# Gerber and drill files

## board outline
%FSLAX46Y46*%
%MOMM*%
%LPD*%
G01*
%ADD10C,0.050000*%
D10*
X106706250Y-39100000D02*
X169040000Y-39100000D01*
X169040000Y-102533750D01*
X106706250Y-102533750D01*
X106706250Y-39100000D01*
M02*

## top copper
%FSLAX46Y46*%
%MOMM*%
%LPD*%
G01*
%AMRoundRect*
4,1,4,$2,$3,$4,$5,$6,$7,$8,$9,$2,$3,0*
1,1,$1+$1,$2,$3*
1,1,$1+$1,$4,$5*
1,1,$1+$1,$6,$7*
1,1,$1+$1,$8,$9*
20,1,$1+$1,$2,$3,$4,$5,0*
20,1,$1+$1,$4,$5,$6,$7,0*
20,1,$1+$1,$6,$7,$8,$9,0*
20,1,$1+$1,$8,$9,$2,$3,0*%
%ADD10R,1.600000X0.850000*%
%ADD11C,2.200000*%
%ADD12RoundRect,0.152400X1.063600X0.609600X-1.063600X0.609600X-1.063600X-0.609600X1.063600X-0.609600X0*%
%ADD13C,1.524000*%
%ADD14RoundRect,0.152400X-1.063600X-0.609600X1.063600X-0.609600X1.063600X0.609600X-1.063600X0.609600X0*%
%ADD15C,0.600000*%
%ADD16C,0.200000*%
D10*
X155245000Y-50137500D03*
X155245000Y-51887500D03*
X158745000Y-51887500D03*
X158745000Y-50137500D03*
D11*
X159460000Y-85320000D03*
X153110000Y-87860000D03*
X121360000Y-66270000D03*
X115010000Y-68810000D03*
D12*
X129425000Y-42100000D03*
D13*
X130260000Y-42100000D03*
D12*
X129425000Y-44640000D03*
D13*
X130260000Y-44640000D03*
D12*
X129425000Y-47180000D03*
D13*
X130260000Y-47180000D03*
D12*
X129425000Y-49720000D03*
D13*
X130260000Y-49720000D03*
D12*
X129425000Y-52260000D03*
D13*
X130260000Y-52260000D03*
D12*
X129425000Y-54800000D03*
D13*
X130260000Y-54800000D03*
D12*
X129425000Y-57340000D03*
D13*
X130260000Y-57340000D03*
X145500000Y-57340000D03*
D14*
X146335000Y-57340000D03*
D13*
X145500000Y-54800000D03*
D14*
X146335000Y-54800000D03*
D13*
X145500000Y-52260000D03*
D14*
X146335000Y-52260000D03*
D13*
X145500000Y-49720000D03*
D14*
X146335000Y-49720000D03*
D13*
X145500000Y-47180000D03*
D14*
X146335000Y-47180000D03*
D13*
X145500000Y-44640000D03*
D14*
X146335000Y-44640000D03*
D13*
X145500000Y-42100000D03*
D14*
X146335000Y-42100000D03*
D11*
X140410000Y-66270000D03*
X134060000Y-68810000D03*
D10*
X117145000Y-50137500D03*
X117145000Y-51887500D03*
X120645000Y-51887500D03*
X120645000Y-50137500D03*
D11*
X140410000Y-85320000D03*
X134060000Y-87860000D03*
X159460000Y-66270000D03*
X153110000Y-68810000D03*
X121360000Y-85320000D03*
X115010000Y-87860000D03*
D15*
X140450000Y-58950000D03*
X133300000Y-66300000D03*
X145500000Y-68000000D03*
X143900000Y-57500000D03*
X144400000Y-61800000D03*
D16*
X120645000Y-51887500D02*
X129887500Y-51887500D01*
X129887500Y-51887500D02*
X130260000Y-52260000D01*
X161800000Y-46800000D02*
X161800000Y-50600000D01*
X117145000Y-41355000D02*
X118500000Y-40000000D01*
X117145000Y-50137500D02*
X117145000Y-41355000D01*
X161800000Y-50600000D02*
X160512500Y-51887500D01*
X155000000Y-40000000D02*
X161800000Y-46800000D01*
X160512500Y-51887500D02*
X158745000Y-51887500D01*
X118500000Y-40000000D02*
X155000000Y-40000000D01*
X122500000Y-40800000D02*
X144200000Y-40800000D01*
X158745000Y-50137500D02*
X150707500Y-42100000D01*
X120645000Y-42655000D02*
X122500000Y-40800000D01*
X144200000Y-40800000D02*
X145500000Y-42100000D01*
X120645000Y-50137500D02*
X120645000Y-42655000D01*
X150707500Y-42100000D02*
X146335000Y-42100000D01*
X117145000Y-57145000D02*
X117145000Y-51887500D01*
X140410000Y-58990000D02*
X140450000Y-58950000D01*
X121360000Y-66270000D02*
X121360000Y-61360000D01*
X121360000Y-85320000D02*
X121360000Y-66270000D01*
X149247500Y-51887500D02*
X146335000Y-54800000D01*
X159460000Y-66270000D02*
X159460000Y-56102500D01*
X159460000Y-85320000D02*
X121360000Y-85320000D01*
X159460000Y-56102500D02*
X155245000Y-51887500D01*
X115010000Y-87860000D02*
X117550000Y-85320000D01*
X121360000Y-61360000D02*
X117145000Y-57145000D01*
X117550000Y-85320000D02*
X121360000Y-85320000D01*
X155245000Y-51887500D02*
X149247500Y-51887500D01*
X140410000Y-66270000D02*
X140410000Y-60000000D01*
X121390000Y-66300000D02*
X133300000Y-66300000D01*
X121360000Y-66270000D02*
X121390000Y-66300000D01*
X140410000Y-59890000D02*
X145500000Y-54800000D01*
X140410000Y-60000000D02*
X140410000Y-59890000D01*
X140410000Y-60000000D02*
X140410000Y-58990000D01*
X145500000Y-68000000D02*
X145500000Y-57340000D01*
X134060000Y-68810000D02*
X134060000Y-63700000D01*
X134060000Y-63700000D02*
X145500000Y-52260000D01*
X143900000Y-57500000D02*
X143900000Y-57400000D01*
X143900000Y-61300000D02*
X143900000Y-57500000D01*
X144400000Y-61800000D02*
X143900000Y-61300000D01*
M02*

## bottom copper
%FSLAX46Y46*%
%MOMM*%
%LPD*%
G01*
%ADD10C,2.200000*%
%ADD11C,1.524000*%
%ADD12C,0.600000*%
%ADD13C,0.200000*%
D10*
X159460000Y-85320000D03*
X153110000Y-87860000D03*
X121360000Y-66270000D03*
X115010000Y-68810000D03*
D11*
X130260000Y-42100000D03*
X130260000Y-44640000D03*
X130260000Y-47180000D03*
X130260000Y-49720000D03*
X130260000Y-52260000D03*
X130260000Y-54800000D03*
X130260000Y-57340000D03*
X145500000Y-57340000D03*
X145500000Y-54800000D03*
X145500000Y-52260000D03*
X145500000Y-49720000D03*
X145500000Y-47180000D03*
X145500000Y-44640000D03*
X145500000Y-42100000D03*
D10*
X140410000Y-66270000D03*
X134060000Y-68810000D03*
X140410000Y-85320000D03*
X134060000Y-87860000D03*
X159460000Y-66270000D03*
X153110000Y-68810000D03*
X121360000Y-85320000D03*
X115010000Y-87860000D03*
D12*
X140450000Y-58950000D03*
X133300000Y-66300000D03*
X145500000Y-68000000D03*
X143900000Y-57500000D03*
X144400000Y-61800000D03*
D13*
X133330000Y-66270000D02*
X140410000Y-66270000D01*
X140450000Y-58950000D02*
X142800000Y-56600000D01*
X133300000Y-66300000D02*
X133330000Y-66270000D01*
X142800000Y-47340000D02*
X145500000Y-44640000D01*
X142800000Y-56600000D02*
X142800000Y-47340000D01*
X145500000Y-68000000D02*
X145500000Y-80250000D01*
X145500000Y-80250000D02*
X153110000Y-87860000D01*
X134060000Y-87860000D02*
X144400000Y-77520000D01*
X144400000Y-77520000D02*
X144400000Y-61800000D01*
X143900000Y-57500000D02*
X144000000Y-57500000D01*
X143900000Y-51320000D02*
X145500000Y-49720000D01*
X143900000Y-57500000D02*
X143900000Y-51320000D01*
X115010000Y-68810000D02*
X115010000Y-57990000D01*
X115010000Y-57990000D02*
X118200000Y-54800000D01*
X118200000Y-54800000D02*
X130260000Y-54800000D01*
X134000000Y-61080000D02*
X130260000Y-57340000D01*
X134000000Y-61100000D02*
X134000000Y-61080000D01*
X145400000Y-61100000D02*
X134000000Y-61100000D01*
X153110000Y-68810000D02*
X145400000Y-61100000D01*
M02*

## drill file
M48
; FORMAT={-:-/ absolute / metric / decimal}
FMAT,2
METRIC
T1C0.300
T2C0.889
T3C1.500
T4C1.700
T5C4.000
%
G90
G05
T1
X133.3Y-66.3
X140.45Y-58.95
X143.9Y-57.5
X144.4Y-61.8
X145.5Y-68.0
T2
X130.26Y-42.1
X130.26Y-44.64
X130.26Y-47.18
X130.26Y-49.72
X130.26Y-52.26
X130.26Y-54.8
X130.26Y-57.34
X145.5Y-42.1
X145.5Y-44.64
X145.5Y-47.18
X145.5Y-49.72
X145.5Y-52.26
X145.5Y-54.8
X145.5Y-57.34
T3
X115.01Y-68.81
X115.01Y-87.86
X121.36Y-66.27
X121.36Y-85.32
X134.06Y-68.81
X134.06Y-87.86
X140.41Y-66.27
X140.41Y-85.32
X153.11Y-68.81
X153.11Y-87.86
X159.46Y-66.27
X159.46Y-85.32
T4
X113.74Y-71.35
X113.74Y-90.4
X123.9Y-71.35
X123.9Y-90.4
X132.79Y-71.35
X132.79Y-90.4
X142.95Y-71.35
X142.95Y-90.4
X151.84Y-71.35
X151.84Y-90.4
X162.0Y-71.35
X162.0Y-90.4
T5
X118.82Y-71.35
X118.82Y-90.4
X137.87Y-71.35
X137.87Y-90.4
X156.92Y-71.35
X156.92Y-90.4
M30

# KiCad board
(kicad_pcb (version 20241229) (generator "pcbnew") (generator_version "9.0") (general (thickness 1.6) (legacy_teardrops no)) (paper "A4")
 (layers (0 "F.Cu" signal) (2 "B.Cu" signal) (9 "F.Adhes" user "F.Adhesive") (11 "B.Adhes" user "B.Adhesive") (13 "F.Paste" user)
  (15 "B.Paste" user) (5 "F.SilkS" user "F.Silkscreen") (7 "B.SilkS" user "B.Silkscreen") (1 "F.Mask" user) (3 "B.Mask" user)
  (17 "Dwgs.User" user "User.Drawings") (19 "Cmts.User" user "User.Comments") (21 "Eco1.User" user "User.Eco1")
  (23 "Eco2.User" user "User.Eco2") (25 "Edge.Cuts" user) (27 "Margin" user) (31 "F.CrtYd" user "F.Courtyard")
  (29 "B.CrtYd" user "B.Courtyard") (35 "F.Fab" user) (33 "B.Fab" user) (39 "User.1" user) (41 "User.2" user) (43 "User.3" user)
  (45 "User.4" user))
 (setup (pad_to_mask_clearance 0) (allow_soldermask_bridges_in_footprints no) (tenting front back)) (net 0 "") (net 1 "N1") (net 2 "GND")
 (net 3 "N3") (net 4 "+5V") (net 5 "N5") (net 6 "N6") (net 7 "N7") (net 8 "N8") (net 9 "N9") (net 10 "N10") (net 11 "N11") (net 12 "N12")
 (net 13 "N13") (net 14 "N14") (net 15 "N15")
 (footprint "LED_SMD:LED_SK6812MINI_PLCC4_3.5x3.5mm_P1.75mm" (layer "F.Cu") (at 156.995 51.0125)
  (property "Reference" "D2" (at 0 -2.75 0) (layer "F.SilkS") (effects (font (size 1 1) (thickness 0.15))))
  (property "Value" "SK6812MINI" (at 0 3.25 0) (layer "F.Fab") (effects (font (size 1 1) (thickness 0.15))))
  (pad "1" smd rect (at -1.75 -0.875) (size 1.6 0.85) (layers "F.Cu" "F.Mask" "F.Paste") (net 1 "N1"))
  (pad "2" smd rect (at -1.75 0.875) (size 1.6 0.85) (layers "F.Cu" "F.Mask" "F.Paste") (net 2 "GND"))
  (pad "3" smd rect (at 1.75 0.875) (size 1.6 0.85) (layers "F.Cu" "F.Mask" "F.Paste") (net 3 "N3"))
  (pad "4" smd rect (at 1.75 -0.875) (size 1.6 0.85) (layers "F.Cu" "F.Mask" "F.Paste") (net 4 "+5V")))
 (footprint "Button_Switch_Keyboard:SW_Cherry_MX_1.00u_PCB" (layer "F.Cu") (at 159.46 85.32)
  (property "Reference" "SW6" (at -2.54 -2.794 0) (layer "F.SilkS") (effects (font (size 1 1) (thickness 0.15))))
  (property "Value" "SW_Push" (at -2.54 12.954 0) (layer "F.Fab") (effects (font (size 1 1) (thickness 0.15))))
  (pad "" np_thru_hole circle (at -7.62 5.08) (size 1.7 1.7) (drill 1.7) (layers "*.Cu" "*.Mask"))
  (pad "" np_thru_hole circle (at -2.54 5.08) (size 4 4) (drill 4) (layers "*.Cu" "*.Mask"))
  (pad "" np_thru_hole circle (at 2.54 5.08) (size 1.7 1.7) (drill 1.7) (layers "*.Cu" "*.Mask"))
  (pad "1" thru_hole circle (at 0 0) (size 2.2 2.2) (drill 1.5) (layers "*.Cu" "*.Mask") (remove_unused_layers no) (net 2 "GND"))
  (pad "2" thru_hole circle (at -6.35 2.54) (size 2.2 2.2) (drill 1.5) (layers "*.Cu" "*.Mask") (remove_unused_layers no) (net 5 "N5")))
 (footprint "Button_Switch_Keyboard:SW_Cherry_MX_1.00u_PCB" (layer "F.Cu") (at 121.36 66.27)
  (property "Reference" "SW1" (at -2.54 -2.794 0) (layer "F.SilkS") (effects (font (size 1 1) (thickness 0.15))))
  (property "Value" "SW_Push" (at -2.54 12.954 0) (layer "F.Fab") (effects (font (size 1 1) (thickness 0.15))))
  (pad "" np_thru_hole circle (at -7.62 5.08) (size 1.7 1.7) (drill 1.7) (layers "*.Cu" "*.Mask"))
  (pad "" np_thru_hole circle (at -2.54 5.08) (size 4 4) (drill 4) (layers "*.Cu" "*.Mask"))
  (pad "" np_thru_hole circle (at 2.54 5.08) (size 1.7 1.7) (drill 1.7) (layers "*.Cu" "*.Mask"))
  (pad "1" thru_hole circle (at 0 0) (size 2.2 2.2) (drill 1.5) (layers "*.Cu" "*.Mask") (remove_unused_layers no) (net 2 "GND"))
  (pad "2" thru_hole circle (at -6.35 2.54) (size 2.2 2.2) (drill 1.5) (layers "*.Cu" "*.Mask") (remove_unused_layers no) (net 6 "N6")))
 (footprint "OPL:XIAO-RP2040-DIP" (layer "F.Cu") (at 137.88 49.72)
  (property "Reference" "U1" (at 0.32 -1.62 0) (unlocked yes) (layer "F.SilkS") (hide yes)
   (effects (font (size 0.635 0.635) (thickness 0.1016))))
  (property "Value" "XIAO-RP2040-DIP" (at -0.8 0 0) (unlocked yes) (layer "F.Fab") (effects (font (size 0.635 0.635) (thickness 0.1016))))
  (pad "1" smd roundrect (at -8.455 -7.62 180) (size 2.432 1.524) (layers "F.Cu" "F.Mask") (roundrect_rratio 0.1) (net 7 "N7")
   (thermal_bridge_angle 45))
  (pad "1" thru_hole circle (at -7.62 -7.62 180) (size 1.524 1.524) (drill 0.889) (layers "*.Cu" "*.Mask") (remove_unused_layers no)
   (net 7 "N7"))
  (pad "2" smd roundrect (at -8.455 -5.08 180) (size 2.432 1.524) (layers "F.Cu" "F.Mask") (roundrect_rratio 0.1) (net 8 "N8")
   (thermal_bridge_angle 45))
  (pad "2" thru_hole circle (at -7.62 -5.08 180) (size 1.524 1.524) (drill 0.889) (layers "*.Cu" "*.Mask") (remove_unused_layers no)
   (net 8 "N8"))
  (pad "3" smd roundrect (at -8.455 -2.54 180) (size 2.432 1.524) (layers "F.Cu" "F.Mask") (roundrect_rratio 0.1) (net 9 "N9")
   (thermal_bridge_angle 45))
  (pad "3" thru_hole circle (at -7.62 -2.54 180) (size 1.524 1.524) (drill 0.889) (layers "*.Cu" "*.Mask") (remove_unused_layers no)
   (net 9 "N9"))
  (pad "4" smd roundrect (at -8.455 0 180) (size 2.432 1.524) (layers "F.Cu" "F.Mask") (roundrect_rratio 0.1) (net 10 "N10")
   (thermal_bridge_angle 45))
  (pad "4" thru_hole circle (at -7.62 0 180) (size 1.524 1.524) (drill 0.889) (layers "*.Cu" "*.Mask") (remove_unused_layers no)
   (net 10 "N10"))
  (pad "5" smd roundrect (at -8.455 2.54 180) (size 2.432 1.524) (layers "F.Cu" "F.Mask") (roundrect_rratio 0.1) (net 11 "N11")
   (thermal_bridge_angle 45))
  (pad "5" thru_hole circle (at -7.62 2.54 180) (size 1.524 1.524) (drill 0.889) (layers "*.Cu" "*.Mask") (remove_unused_layers no)
   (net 11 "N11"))
  (pad "6" smd roundrect (at -8.455 5.08 180) (size 2.432 1.524) (layers "F.Cu" "F.Mask") (roundrect_rratio 0.1) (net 6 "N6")
   (thermal_bridge_angle 45))
  (pad "6" thru_hole circle (at -7.62 5.08 180) (size 1.524 1.524) (drill 0.889) (layers "*.Cu" "*.Mask") (remove_unused_layers no)
   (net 6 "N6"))
  (pad "7" smd roundrect (at -8.455 7.62 180) (size 2.432 1.524) (layers "F.Cu" "F.Mask") (roundrect_rratio 0.1) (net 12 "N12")
   (thermal_bridge_angle 45))
  (pad "7" thru_hole circle (at -7.62 7.62 180) (size 1.524 1.524) (drill 0.889) (layers "*.Cu" "*.Mask") (remove_unused_layers no)
   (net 12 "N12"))
  (pad "8" thru_hole circle (at 7.62 7.62) (size 1.524 1.524) (drill 0.889) (layers "*.Cu" "*.Mask") (remove_unused_layers no) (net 5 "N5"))
  (pad "8" smd roundrect (at 8.455 7.62) (size 2.432 1.524) (layers "F.Cu" "F.Mask") (roundrect_rratio 0.1) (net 5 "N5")
   (thermal_bridge_angle 45))
  (pad "9" thru_hole circle (at 7.62 5.08) (size 1.524 1.524) (drill 0.889) (layers "*.Cu" "*.Mask") (remove_unused_layers no) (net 2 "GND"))
  (pad "9" smd roundrect (at 8.455 5.08) (size 2.432 1.524) (layers "F.Cu" "F.Mask") (roundrect_rratio 0.1) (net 2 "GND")
   (thermal_bridge_angle 45))
  (pad "10" thru_hole circle (at 7.62 2.54) (size 1.524 1.524) (drill 0.889) (layers "*.Cu" "*.Mask") (remove_unused_layers no)
   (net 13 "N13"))
  (pad "10" smd roundrect (at 8.455 2.54) (size 2.432 1.524) (layers "F.Cu" "F.Mask") (roundrect_rratio 0.1) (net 13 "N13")
   (thermal_bridge_angle 45))
  (pad "11" thru_hole circle (at 7.62 0) (size 1.524 1.524) (drill 0.889) (layers "*.Cu" "*.Mask") (remove_unused_layers no) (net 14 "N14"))
  (pad "11" smd roundrect (at 8.455 0) (size 2.432 1.524) (layers "F.Cu" "F.Mask") (roundrect_rratio 0.1) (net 14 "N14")
   (thermal_bridge_angle 45))
  (pad "12" thru_hole circle (at 7.62 -2.54) (size 1.524 1.524) (drill 0.889) (layers "*.Cu" "*.Mask") (remove_unused_layers no)
   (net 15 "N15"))
  (pad "12" smd roundrect (at 8.455 -2.54) (size 2.432 1.524) (layers "F.Cu" "F.Mask") (roundrect_rratio 0.1) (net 15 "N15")
   (thermal_bridge_angle 45))
  (pad "13" thru_hole circle (at 7.62 -5.08) (size 1.524 1.524) (drill 0.889) (layers "*.Cu" "*.Mask") (remove_unused_layers no)
   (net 2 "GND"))
  (pad "13" smd roundrect (at 8.455 -5.08) (size 2.432 1.524) (layers "F.Cu" "F.Mask") (roundrect_rratio 0.1) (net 2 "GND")
   (thermal_bridge_angle 45))
  (pad "14" thru_hole circle (at 7.62 -7.62) (size 1.524 1.524) (drill 0.889) (layers "*.Cu" "*.Mask") (remove_unused_layers no)
   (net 4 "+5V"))
  (pad "14" smd roundrect (at 8.455 -7.62) (size 2.432 1.524) (layers "F.Cu" "F.Mask") (roundrect_rratio 0.1) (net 4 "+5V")
   (thermal_bridge_angle 45)))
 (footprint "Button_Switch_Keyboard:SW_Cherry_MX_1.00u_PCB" (layer "F.Cu") (at 140.41 66.27)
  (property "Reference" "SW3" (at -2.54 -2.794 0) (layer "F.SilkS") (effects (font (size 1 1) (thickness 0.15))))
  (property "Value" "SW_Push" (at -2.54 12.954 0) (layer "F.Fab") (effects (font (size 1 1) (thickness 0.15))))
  (pad "" np_thru_hole circle (at -7.62 5.08) (size 1.7 1.7) (drill 1.7) (layers "*.Cu" "*.Mask"))
  (pad "" np_thru_hole circle (at -2.54 5.08) (size 4 4) (drill 4) (layers "*.Cu" "*.Mask"))
  (pad "" np_thru_hole circle (at 2.54 5.08) (size 1.7 1.7) (drill 1.7) (layers "*.Cu" "*.Mask"))
  (pad "1" thru_hole circle (at 0 0) (size 2.2 2.2) (drill 1.5) (layers "*.Cu" "*.Mask") (remove_unused_layers no) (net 2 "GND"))
  (pad "2" thru_hole circle (at -6.35 2.54) (size 2.2 2.2) (drill 1.5) (layers "*.Cu" "*.Mask") (remove_unused_layers no) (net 13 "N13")))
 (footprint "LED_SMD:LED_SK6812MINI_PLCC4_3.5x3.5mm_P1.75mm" (layer "F.Cu") (at 118.895 51.0125)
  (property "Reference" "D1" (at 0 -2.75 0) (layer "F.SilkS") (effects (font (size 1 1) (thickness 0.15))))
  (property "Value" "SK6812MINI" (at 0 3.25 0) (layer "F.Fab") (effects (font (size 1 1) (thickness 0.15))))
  (pad "1" smd rect (at -1.75 -0.875) (size 1.6 0.85) (layers "F.Cu" "F.Mask" "F.Paste") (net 3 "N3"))
  (pad "2" smd rect (at -1.75 0.875) (size 1.6 0.85) (layers "F.Cu" "F.Mask" "F.Paste") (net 2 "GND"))
  (pad "3" smd rect (at 1.75 0.875) (size 1.6 0.85) (layers "F.Cu" "F.Mask" "F.Paste") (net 11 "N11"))
  (pad "4" smd rect (at 1.75 -0.875) (size 1.6 0.85) (layers "F.Cu" "F.Mask" "F.Paste") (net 4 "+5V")))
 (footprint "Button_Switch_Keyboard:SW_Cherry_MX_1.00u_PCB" (layer "F.Cu") (at 140.41 85.32)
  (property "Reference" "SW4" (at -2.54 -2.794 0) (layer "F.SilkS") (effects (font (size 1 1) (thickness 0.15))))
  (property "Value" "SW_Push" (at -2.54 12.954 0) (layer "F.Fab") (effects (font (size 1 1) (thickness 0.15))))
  (pad "" np_thru_hole circle (at -7.62 5.08) (size 1.7 1.7) (drill 1.7) (layers "*.Cu" "*.Mask"))
  (pad "" np_thru_hole circle (at -2.54 5.08) (size 4 4) (drill 4) (layers "*.Cu" "*.Mask"))
  (pad "" np_thru_hole circle (at 2.54 5.08) (size 1.7 1.7) (drill 1.7) (layers "*.Cu" "*.Mask"))
  (pad "1" thru_hole circle (at 0 0) (size 2.2 2.2) (drill 1.5) (layers "*.Cu" "*.Mask") (remove_unused_layers no) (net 2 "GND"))
  (pad "2" thru_hole circle (at -6.35 2.54) (size 2.2 2.2) (drill 1.5) (layers "*.Cu" "*.Mask") (remove_unused_layers no) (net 14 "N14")))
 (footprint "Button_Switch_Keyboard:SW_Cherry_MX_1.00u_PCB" (layer "F.Cu") (at 159.46 66.27)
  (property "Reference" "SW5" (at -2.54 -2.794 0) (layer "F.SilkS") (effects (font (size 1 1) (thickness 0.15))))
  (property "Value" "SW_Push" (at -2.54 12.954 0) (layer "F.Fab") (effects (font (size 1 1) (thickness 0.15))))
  (pad "" np_thru_hole circle (at -7.62 5.08) (size 1.7 1.7) (drill 1.7) (layers "*.Cu" "*.Mask"))
  (pad "" np_thru_hole circle (at -2.54 5.08) (size 4 4) (drill 4) (layers "*.Cu" "*.Mask"))
  (pad "" np_thru_hole circle (at 2.54 5.08) (size 1.7 1.7) (drill 1.7) (layers "*.Cu" "*.Mask"))
  (pad "1" thru_hole circle (at 0 0) (size 2.2 2.2) (drill 1.5) (layers "*.Cu" "*.Mask") (remove_unused_layers no) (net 2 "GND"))
  (pad "2" thru_hole circle (at -6.35 2.54) (size 2.2 2.2) (drill 1.5) (layers "*.Cu" "*.Mask") (remove_unused_layers no) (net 12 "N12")))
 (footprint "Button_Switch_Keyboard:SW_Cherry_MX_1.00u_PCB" (layer "F.Cu") (at 121.36 85.32)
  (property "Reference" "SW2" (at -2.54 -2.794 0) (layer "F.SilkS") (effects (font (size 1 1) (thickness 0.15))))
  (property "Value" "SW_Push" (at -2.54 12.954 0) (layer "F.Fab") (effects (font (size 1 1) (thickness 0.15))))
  (pad "" np_thru_hole circle (at -7.62 5.08) (size 1.7 1.7) (drill 1.7) (layers "*.Cu" "*.Mask"))
  (pad "" np_thru_hole circle (at -2.54 5.08) (size 4 4) (drill 4) (layers "*.Cu" "*.Mask"))
  (pad "" np_thru_hole circle (at 2.54 5.08) (size 1.7 1.7) (drill 1.7) (layers "*.Cu" "*.Mask"))
  (pad "1" thru_hole circle (at 0 0) (size 2.2 2.2) (drill 1.5) (layers "*.Cu" "*.Mask") (remove_unused_layers no) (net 2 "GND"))
  (pad "2" thru_hole circle (at -6.35 2.54) (size 2.2 2.2) (drill 1.5) (layers "*.Cu" "*.Mask") (remove_unused_layers no) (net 2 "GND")))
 (gr_rect (start 106.70625 39.1) (end 169.04 102.53375) (stroke (width 0.05) (type default)) (fill no) (layer "Edge.Cuts"))
 (segment (start 120.645 51.8875) (end 129.8875 51.8875) (width 0.2) (layer "F.Cu") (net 11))
 (segment (start 129.8875 51.8875) (end 130.26 52.26) (width 0.2) (layer "F.Cu") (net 11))
 (segment (start 161.8 46.8) (end 161.8 50.6) (width 0.2) (layer "F.Cu") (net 3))
 (segment (start 117.145 41.355) (end 118.5 40) (width 0.2) (layer "F.Cu") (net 3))
 (segment (start 117.145 50.1375) (end 117.145 41.355) (width 0.2) (layer "F.Cu") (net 3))
 (segment (start 161.8 50.6) (end 160.5125 51.8875) (width 0.2) (layer "F.Cu") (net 3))
 (segment (start 155 40) (end 161.8 46.8) (width 0.2) (layer "F.Cu") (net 3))
 (segment (start 160.5125 51.8875) (end 158.745 51.8875) (width 0.2) (layer "F.Cu") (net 3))
 (segment (start 118.5 40) (end 155 40) (width 0.2) (layer "F.Cu") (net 3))
 (segment (start 122.5 40.8) (end 144.2 40.8) (width 0.2) (layer "F.Cu") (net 4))
 (segment (start 158.745 50.1375) (end 150.7075 42.1) (width 0.2) (layer "F.Cu") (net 4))
 (segment (start 120.645 42.655) (end 122.5 40.8) (width 0.2) (layer "F.Cu") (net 4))
 (segment (start 144.2 40.8) (end 145.5 42.1) (width 0.2) (layer "F.Cu") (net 4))
 (segment (start 120.645 50.1375) (end 120.645 42.655) (width 0.2) (layer "F.Cu") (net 4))
 (segment (start 150.7075 42.1) (end 146.335 42.1) (width 0.2) (layer "F.Cu") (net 4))
 (segment (start 117.145 57.145) (end 117.145 51.8875) (width 0.2) (layer "F.Cu") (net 2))
 (segment (start 140.41 58.99) (end 140.45 58.95) (width 0.2) (layer "F.Cu") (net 2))
 (segment (start 121.36 66.27) (end 121.36 61.36) (width 0.2) (layer "F.Cu") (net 2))
 (segment (start 121.36 85.32) (end 121.36 66.27) (width 0.2) (layer "F.Cu") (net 2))
 (segment (start 149.2475 51.8875) (end 146.335 54.8) (width 0.2) (layer "F.Cu") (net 2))
 (segment (start 159.46 66.27) (end 159.46 56.1025) (width 0.2) (layer "F.Cu") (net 2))
 (segment (start 159.46 85.32) (end 121.36 85.32) (width 0.2) (layer "F.Cu") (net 2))
 (segment (start 159.46 56.1025) (end 155.245 51.8875) (width 0.2) (layer "F.Cu") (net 2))
 (segment (start 115.01 87.86) (end 117.55 85.32) (width 0.2) (layer "F.Cu") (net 2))
 (segment (start 121.36 61.36) (end 117.145 57.145) (width 0.2) (layer "F.Cu") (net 2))
 (segment (start 117.55 85.32) (end 121.36 85.32) (width 0.2) (layer "F.Cu") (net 2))
 (segment (start 155.245 51.8875) (end 149.2475 51.8875) (width 0.2) (layer "F.Cu") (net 2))
 (segment (start 140.41 66.27) (end 140.41 60) (width 0.2) (layer "F.Cu") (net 2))
 (segment (start 121.39 66.3) (end 133.3 66.3) (width 0.2) (layer "F.Cu") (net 2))
 (segment (start 121.36 66.27) (end 121.39 66.3) (width 0.2) (layer "F.Cu") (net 2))
 (segment (start 140.41 59.89) (end 145.5 54.8) (width 0.2) (layer "F.Cu") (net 2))
 (segment (start 140.41 60) (end 140.41 59.89) (width 0.2) (layer "F.Cu") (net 2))
 (segment (start 140.41 60) (end 140.41 58.99) (width 0.2) (layer "F.Cu") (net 2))
 (via (at 140.45 58.95) (size 0.6) (drill 0.3) (layers "F.Cu" "B.Cu") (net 2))
 (via (at 133.3 66.3) (size 0.6) (drill 0.3) (layers "F.Cu" "B.Cu") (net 2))
 (segment (start 133.33 66.27) (end 140.41 66.27) (width 0.2) (layer "B.Cu") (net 2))
 (segment (start 140.45 58.95) (end 142.8 56.6) (width 0.2) (layer "B.Cu") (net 2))
 (segment (start 133.3 66.3) (end 133.33 66.27) (width 0.2) (layer "B.Cu") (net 2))
 (segment (start 142.8 47.34) (end 145.5 44.64) (width 0.2) (layer "B.Cu") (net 2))
 (segment (start 142.8 56.6) (end 142.8 47.34) (width 0.2) (layer "B.Cu") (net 2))
 (segment (start 145.5 68) (end 145.5 57.34) (width 0.2) (layer "F.Cu") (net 5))
 (via (at 145.5 68) (size 0.6) (drill 0.3) (layers "F.Cu" "B.Cu") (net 5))
 (segment (start 145.5 68) (end 145.5 80.25) (width 0.2) (layer "B.Cu") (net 5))
 (segment (start 145.5 80.25) (end 153.11 87.86) (width 0.2) (layer "B.Cu") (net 5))
 (segment (start 134.06 68.81) (end 134.06 63.7) (width 0.2) (layer "F.Cu") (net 13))
 (segment (start 134.06 63.7) (end 145.5 52.26) (width 0.2) (layer "F.Cu") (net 13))
 (segment (start 143.9 57.5) (end 143.9 57.4) (width 0.2) (layer "F.Cu") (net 14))
 (segment (start 143.9 61.3) (end 143.9 57.5) (width 0.2) (layer "F.Cu") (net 14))
 (segment (start 144.4 61.8) (end 143.9 61.3) (width 0.2) (layer "F.Cu") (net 14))
 (via (at 143.9 57.5) (size 0.6) (drill 0.3) (layers "F.Cu" "B.Cu") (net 14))
 (via (at 144.4 61.8) (size 0.6) (drill 0.3) (layers "F.Cu" "B.Cu") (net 14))
 (segment (start 134.06 87.86) (end 144.4 77.52) (width 0.2) (layer "B.Cu") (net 14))
 (segment (start 144.4 77.52) (end 144.4 61.8) (width 0.2) (layer "B.Cu") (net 14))
 (segment (start 143.9 57.5) (end 144 57.5) (width 0.2) (layer "B.Cu") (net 14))
 (segment (start 143.9 51.32) (end 145.5 49.72) (width 0.2) (layer "B.Cu") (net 14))
 (segment (start 143.9 57.5) (end 143.9 51.32) (width 0.2) (layer "B.Cu") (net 14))
 (segment (start 115.01 68.81) (end 115.01 57.99) (width 0.2) (layer "B.Cu") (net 6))
 (segment (start 115.01 57.99) (end 118.2 54.8) (width 0.2) (layer "B.Cu") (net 6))
 (segment (start 118.2 54.8) (end 130.26 54.8) (width 0.2) (layer "B.Cu") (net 6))
 (segment (start 134 61.08) (end 130.26 57.34) (width 0.2) (layer "B.Cu") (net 12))
 (segment (start 134 61.1) (end 134 61.08) (width 0.2) (layer "B.Cu") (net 12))
 (segment (start 145.4 61.1) (end 134 61.1) (width 0.2) (layer "B.Cu") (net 12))
 (segment (start 153.11 68.81) (end 145.4 61.1) (width 0.2) (layer "B.Cu") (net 12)))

